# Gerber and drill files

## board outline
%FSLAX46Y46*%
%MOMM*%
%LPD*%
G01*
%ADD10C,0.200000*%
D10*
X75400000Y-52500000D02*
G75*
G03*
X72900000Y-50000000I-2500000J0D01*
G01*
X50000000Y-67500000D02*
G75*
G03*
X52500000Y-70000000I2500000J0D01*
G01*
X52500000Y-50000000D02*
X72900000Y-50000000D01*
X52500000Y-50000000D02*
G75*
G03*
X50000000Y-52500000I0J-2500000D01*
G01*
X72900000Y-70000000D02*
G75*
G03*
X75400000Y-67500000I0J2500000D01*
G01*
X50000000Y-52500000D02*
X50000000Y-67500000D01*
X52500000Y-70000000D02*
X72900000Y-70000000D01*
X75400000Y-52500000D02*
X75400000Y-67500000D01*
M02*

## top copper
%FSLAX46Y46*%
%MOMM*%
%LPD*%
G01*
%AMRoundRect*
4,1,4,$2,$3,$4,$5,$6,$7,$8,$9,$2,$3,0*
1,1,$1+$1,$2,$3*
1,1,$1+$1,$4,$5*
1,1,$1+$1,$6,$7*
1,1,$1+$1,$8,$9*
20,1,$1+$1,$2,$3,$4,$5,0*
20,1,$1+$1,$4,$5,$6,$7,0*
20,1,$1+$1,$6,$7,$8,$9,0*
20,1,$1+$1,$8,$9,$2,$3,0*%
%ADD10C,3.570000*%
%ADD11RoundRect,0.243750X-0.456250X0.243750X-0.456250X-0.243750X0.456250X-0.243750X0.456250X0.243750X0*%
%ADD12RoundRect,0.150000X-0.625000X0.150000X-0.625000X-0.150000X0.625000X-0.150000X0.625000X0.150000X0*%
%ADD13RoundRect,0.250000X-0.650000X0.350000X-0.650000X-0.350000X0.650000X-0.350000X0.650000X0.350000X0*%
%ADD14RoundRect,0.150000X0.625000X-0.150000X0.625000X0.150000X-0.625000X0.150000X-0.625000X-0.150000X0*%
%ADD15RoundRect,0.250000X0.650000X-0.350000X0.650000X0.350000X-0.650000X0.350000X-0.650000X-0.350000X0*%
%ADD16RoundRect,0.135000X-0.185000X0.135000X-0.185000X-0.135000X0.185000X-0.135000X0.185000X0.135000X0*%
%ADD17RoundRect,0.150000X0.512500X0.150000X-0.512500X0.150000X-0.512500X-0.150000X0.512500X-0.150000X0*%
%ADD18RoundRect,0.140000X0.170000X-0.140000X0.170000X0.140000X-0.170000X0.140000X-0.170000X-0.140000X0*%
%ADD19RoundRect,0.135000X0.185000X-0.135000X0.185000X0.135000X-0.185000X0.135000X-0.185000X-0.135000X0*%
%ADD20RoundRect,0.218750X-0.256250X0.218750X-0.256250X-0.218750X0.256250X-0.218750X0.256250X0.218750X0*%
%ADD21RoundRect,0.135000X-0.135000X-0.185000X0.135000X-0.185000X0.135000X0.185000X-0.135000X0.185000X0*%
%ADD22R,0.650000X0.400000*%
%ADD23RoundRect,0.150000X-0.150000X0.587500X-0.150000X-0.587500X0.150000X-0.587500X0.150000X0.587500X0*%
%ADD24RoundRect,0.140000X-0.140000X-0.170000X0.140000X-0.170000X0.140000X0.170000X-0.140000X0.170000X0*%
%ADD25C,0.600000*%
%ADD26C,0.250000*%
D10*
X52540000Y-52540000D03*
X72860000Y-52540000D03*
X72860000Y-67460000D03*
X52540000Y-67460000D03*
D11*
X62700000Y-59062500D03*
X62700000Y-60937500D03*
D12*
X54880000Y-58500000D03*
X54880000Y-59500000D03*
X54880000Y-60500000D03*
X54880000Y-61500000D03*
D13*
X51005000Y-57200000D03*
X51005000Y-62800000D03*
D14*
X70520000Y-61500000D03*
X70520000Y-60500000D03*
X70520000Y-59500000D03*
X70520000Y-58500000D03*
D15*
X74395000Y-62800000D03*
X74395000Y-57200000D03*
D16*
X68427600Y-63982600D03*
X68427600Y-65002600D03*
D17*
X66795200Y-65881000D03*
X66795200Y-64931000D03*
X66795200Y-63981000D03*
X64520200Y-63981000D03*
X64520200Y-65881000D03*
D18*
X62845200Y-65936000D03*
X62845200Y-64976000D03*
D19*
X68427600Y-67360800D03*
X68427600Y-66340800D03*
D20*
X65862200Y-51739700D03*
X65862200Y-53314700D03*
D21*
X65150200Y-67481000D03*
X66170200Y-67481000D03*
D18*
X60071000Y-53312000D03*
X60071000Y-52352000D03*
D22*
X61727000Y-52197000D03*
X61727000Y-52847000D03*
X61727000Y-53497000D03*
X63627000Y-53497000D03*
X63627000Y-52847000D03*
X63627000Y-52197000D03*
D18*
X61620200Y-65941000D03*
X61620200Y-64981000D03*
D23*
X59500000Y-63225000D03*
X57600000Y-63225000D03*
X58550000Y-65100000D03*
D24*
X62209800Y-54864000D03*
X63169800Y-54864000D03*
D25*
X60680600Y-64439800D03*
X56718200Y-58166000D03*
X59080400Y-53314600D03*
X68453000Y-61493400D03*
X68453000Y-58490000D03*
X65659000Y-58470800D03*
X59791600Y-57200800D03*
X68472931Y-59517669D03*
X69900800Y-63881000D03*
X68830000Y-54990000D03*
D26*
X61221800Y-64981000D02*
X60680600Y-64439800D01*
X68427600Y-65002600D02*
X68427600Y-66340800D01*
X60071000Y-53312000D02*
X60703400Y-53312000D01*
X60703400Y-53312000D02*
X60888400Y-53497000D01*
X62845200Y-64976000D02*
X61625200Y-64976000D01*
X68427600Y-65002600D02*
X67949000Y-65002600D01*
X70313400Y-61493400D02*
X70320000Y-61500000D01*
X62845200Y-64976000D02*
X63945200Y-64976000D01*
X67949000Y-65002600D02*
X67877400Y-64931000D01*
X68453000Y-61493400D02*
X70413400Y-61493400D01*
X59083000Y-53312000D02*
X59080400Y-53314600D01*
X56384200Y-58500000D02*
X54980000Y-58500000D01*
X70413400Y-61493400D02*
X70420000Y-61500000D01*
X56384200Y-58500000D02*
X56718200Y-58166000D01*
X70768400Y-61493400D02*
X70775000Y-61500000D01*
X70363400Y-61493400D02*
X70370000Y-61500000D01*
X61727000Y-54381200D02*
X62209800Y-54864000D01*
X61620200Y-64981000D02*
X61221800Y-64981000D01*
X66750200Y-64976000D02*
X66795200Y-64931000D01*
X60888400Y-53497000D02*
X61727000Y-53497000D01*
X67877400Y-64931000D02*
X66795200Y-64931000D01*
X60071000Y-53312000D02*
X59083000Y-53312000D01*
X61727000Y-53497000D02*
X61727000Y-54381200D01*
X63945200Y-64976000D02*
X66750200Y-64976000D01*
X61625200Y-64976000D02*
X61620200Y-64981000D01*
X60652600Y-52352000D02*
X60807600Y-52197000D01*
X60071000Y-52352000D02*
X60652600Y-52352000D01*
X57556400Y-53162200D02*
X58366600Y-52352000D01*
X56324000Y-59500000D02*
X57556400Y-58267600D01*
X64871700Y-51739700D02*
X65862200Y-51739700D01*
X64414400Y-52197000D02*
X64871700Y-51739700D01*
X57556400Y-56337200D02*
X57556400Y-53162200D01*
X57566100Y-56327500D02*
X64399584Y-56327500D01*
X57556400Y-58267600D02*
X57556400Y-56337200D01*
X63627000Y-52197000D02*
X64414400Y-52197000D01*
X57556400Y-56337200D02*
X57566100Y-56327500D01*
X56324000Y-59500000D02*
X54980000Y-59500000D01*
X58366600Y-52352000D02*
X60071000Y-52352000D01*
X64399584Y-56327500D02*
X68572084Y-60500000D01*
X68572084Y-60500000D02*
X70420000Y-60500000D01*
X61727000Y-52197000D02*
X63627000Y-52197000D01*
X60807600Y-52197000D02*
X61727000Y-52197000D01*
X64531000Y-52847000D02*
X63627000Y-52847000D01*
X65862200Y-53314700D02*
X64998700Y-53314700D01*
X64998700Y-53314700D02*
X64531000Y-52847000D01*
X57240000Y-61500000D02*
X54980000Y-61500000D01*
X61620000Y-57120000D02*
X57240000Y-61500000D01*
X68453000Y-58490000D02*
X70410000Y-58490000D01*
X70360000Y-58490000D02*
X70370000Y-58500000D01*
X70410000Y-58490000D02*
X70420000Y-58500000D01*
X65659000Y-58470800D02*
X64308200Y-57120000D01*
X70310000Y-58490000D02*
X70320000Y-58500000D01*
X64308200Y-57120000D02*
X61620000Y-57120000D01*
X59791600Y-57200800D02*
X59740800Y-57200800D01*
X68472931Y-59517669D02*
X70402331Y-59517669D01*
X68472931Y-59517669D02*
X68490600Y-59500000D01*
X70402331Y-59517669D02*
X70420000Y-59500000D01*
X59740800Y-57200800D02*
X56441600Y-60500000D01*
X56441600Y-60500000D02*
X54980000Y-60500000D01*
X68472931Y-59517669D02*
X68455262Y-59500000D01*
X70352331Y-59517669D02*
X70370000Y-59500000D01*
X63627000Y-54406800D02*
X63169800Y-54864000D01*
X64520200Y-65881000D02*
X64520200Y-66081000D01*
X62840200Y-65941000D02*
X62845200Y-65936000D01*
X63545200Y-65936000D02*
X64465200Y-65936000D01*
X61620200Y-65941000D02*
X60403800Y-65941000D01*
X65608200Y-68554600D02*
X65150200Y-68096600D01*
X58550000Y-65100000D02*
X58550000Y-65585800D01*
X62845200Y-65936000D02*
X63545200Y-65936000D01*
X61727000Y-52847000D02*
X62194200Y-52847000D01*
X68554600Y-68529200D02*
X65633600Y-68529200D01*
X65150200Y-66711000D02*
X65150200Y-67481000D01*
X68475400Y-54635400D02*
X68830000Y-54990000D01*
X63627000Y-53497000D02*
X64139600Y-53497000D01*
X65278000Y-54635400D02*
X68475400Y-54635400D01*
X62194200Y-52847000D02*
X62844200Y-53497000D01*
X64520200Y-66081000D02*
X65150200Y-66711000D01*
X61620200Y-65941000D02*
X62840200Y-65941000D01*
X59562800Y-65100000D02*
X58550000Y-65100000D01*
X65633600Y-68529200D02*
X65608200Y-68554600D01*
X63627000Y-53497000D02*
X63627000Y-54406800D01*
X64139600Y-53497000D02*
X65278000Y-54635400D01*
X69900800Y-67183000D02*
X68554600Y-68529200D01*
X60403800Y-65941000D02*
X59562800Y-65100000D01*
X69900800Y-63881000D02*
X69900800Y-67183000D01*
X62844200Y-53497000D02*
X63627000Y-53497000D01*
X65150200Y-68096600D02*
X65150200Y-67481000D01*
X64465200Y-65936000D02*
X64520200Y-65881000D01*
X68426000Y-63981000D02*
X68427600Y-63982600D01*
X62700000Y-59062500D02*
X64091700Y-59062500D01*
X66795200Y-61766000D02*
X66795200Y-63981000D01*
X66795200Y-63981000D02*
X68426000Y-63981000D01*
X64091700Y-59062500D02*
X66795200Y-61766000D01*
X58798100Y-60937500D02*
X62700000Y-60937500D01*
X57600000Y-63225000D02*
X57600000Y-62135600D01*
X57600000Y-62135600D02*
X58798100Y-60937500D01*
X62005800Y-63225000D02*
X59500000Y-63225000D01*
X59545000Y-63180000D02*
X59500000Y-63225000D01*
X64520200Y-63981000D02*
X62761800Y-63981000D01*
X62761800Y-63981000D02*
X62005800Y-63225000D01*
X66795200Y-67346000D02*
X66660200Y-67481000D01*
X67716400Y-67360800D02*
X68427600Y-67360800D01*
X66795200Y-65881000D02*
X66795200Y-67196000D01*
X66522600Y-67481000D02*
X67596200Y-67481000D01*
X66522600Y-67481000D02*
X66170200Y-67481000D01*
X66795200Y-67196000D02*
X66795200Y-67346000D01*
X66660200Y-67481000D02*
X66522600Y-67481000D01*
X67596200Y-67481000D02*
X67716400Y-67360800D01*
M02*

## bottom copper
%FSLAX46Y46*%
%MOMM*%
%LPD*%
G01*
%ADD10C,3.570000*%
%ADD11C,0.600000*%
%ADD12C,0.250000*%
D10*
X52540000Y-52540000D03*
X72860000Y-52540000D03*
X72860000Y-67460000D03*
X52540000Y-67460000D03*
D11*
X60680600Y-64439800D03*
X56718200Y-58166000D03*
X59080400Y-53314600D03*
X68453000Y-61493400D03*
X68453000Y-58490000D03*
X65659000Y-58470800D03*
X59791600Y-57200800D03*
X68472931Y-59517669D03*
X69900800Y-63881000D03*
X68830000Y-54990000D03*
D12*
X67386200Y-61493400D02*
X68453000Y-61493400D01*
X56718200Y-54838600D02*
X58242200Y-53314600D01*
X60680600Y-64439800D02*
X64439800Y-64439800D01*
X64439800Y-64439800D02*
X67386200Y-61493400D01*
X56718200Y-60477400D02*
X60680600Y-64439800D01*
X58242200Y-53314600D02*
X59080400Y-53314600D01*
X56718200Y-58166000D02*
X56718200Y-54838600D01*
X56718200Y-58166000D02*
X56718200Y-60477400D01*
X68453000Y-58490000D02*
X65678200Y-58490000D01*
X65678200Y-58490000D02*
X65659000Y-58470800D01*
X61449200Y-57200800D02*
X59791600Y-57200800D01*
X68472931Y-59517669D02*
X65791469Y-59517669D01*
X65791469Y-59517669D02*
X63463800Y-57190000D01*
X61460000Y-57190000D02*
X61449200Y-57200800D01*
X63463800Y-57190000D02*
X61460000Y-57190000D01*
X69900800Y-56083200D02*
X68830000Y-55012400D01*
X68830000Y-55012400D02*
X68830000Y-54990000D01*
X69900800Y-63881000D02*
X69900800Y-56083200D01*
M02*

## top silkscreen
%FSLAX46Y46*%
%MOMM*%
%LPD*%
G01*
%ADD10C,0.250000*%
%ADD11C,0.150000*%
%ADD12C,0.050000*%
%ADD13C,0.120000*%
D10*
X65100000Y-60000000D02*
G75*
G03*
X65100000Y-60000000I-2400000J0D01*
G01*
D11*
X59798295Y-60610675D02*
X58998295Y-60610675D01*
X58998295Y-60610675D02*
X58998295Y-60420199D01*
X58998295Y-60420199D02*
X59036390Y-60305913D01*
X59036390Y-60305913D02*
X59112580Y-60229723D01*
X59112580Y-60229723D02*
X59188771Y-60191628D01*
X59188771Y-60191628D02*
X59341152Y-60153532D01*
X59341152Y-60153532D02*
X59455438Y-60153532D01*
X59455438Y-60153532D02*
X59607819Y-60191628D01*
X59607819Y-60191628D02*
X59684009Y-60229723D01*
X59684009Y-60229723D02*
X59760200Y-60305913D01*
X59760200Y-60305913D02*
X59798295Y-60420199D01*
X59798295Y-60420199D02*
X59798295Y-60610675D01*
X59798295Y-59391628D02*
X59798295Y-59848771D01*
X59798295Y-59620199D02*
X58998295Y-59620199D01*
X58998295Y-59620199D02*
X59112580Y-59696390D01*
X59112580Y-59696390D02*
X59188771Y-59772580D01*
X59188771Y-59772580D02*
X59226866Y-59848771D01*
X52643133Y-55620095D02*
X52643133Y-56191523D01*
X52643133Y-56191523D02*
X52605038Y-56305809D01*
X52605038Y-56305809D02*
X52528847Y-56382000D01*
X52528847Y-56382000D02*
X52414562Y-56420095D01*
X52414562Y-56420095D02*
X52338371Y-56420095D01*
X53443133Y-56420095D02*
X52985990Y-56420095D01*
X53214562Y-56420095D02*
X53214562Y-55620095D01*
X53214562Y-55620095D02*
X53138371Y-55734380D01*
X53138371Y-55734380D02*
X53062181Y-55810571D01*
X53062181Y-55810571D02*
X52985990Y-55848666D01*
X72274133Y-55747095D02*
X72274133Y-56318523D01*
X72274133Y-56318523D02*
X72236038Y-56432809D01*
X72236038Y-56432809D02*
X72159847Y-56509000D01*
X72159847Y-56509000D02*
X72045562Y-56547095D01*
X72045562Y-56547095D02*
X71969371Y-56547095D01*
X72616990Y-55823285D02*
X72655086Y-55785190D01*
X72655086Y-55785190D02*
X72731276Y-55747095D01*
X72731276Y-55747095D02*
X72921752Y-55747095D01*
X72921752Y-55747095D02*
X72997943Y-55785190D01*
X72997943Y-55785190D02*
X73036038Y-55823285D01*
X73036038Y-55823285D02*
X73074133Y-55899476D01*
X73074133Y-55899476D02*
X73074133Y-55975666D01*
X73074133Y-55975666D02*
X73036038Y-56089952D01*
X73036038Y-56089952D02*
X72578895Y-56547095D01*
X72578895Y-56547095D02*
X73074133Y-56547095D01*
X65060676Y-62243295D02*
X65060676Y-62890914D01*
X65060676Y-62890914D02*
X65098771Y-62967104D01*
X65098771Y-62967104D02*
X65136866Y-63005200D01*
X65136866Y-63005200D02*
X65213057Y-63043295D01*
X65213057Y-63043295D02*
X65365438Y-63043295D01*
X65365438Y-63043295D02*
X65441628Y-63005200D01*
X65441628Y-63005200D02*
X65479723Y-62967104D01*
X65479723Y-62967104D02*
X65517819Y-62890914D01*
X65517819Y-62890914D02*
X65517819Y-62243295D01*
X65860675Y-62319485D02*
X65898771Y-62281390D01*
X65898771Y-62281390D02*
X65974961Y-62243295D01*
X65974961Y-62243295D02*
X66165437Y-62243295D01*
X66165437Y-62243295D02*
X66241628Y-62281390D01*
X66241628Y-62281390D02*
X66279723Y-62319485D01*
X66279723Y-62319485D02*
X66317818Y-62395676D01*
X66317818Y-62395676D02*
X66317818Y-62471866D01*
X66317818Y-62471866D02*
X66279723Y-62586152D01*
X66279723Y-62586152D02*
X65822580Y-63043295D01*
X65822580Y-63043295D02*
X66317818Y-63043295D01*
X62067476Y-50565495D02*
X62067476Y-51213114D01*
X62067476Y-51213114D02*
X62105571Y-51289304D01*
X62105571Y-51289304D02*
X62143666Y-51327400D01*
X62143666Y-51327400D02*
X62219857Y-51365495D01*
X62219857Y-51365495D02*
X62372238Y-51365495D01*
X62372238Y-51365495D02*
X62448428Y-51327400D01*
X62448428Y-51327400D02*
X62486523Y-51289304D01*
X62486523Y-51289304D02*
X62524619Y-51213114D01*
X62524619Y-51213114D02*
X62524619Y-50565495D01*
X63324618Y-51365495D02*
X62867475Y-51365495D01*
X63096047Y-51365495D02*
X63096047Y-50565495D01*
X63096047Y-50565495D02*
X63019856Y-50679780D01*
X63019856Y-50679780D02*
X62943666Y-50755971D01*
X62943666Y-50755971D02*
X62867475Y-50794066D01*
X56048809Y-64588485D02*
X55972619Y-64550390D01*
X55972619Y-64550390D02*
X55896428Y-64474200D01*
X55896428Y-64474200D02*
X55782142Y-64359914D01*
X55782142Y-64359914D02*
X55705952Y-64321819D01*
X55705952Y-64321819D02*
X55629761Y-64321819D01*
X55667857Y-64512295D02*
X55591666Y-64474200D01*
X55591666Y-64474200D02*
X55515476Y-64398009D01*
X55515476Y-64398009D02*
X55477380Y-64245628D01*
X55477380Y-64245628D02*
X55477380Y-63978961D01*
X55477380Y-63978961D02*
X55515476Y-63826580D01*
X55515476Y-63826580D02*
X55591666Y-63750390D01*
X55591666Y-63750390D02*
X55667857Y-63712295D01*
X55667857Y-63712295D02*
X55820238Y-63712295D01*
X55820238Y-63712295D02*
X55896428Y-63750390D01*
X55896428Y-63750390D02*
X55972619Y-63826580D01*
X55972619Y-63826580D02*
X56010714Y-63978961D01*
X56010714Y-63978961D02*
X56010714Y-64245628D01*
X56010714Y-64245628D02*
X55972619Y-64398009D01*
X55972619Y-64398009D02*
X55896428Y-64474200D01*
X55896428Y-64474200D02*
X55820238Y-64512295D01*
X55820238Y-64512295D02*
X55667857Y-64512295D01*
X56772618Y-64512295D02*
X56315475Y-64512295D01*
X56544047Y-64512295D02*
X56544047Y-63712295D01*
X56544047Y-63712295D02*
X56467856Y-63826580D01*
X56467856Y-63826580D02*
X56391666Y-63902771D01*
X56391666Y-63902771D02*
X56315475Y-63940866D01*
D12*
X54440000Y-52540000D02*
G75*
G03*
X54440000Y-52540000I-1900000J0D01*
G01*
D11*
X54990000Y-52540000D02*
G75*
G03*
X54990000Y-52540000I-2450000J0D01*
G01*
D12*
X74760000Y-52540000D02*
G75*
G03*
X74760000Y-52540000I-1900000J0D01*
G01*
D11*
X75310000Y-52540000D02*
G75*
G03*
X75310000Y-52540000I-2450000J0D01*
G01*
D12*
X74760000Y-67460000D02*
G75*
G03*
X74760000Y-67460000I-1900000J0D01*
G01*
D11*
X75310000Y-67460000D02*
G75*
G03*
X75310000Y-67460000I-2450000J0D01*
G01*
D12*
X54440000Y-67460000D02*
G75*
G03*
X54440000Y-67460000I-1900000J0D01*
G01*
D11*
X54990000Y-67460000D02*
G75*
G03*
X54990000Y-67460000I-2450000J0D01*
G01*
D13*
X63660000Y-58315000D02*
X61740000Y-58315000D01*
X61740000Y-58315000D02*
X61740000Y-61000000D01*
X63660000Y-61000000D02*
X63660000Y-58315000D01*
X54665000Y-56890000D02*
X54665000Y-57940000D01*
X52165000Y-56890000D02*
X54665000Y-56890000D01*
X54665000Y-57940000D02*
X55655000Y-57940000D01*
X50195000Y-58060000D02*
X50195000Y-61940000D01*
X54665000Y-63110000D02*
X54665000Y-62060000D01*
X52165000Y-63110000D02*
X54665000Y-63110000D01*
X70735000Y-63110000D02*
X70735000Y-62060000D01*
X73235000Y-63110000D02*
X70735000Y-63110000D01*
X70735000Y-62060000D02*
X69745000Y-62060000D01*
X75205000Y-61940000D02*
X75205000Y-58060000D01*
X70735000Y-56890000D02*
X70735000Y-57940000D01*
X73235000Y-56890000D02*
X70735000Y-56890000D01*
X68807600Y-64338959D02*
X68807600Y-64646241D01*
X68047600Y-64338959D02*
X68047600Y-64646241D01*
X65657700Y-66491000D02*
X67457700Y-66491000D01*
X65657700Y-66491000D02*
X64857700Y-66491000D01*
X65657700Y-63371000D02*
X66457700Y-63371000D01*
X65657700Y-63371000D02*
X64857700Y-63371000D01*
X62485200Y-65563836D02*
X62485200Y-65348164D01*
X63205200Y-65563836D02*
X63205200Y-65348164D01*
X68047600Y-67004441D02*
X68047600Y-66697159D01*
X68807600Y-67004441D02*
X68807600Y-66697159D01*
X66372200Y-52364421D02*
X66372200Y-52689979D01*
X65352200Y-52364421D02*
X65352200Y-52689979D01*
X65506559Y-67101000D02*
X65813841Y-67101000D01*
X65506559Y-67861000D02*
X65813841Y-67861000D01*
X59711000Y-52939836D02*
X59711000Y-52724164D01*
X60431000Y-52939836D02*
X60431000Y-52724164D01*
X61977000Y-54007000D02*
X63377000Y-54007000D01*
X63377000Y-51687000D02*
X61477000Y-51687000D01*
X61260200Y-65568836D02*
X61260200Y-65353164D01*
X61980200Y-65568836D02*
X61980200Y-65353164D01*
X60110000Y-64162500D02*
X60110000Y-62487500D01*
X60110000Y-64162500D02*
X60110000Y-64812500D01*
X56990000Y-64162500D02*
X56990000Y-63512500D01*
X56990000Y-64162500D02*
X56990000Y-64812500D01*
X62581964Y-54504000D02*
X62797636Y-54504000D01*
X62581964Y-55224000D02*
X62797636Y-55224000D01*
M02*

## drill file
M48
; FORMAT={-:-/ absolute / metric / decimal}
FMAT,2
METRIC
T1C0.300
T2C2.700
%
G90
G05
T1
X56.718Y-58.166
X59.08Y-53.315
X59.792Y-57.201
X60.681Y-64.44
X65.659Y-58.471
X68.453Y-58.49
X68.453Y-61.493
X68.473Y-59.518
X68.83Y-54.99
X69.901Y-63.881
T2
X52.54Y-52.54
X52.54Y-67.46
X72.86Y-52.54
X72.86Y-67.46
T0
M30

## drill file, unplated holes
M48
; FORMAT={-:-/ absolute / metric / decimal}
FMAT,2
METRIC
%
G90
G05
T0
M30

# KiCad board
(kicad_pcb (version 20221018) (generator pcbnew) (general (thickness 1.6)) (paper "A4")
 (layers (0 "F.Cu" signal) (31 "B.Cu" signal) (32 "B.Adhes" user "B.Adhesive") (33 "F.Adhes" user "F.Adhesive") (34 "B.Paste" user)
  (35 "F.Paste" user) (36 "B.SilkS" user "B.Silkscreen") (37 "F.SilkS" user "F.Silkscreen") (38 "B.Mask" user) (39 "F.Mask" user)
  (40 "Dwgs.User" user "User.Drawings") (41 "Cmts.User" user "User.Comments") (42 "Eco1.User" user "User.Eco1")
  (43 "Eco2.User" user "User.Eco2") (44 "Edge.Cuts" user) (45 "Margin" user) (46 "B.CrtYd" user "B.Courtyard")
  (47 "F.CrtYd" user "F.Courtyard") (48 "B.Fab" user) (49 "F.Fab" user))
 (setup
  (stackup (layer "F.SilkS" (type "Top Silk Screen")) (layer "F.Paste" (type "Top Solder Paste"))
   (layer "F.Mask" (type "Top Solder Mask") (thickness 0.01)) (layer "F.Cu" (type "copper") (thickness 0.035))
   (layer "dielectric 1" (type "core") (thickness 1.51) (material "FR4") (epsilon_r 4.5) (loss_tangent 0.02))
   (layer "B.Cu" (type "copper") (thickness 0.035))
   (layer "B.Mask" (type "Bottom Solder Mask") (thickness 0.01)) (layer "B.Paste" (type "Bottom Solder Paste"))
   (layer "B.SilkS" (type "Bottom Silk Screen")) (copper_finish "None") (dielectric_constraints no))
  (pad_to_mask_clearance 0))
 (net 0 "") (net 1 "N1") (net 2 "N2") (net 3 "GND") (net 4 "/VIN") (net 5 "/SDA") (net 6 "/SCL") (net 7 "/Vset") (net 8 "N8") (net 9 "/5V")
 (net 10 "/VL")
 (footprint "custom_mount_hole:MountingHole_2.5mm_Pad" (layer "F.Cu") (at 52.54 52.54)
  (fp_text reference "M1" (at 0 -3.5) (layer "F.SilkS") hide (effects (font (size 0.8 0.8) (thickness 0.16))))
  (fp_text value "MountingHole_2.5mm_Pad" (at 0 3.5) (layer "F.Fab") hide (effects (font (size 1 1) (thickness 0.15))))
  (fp_circle (center 0 0) (end 1.9 0) (stroke (width 0.05) (type solid)) (fill none) (layer "F.SilkS"))
  (fp_circle (center 0 0) (end 2.45 0) (stroke (width 0.15) (type solid)) (fill none) (layer "F.SilkS"))
  (pad "~" thru_hole circle (at 0 0) (size 3.57 3.57) (drill 2.7) (layers "*.Cu" "*.Mask")))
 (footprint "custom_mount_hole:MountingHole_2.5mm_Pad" (layer "F.Cu") (at 72.86 52.54)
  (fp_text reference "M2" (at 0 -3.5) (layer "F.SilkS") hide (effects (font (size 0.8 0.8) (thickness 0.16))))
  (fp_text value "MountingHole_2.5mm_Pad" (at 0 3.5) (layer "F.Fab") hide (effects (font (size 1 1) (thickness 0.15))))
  (fp_circle (center 0 0) (end 1.9 0) (stroke (width 0.05) (type solid)) (fill none) (layer "F.SilkS"))
  (fp_circle (center 0 0) (end 2.45 0) (stroke (width 0.15) (type solid)) (fill none) (layer "F.SilkS"))
  (pad "~" thru_hole circle (at 0 0) (size 3.57 3.57) (drill 2.7) (layers "*.Cu" "*.Mask")))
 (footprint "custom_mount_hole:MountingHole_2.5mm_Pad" (layer "F.Cu") (at 72.86 67.46)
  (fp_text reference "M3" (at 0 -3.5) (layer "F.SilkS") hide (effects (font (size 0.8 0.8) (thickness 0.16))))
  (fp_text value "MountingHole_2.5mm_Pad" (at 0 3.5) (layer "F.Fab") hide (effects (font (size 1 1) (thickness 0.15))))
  (fp_circle (center 0 0) (end 1.9 0) (stroke (width 0.05) (type solid)) (fill none) (layer "F.SilkS"))
  (fp_circle (center 0 0) (end 2.45 0) (stroke (width 0.15) (type solid)) (fill none) (layer "F.SilkS"))
  (pad "~" thru_hole circle (at 0 0) (size 3.57 3.57) (drill 2.7) (layers "*.Cu" "*.Mask")))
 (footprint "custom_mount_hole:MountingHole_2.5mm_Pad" (layer "F.Cu") (at 52.54 67.46)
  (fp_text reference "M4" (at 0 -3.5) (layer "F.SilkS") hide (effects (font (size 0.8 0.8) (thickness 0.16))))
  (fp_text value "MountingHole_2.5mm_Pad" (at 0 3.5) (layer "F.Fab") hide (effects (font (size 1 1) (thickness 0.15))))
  (fp_circle (center 0 0) (end 1.9 0) (stroke (width 0.05) (type solid)) (fill none) (layer "F.SilkS"))
  (fp_circle (center 0 0) (end 2.45 0) (stroke (width 0.15) (type solid)) (fill none) (layer "F.SilkS"))
  (pad "~" thru_hole circle (at 0 0) (size 3.57 3.57) (drill 2.7) (layers "*.Cu" "*.Mask")))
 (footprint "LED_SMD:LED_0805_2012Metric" (layer "F.Cu") (at 62.7 60 -90)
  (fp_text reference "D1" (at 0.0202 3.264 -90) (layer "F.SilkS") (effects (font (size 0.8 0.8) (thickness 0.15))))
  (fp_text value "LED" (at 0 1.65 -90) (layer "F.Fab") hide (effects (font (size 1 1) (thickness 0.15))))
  (fp_line (start -1.685 -0.96) (end -1.685 0.96) (stroke (width 0.12) (type solid)) (layer "F.SilkS"))
  (fp_line (start -1.685 0.96) (end 1 0.96) (stroke (width 0.12) (type solid)) (layer "F.SilkS"))
  (fp_line (start 1 -0.96) (end -1.685 -0.96) (stroke (width 0.12) (type solid)) (layer "F.SilkS"))
  (pad "1" smd roundrect (at -0.9375 0 270) (size 0.975 1.4) (layers "F.Cu" "F.Paste" "F.Mask") (roundrect_rratio 0.25) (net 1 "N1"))
  (pad "2" smd roundrect (at 0.9375 0 270) (size 0.975 1.4) (layers "F.Cu" "F.Paste" "F.Mask") (roundrect_rratio 0.25) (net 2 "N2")))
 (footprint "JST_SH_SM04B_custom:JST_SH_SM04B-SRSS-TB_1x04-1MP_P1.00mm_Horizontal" (layer "F.Cu") (at 52.88 60 -90)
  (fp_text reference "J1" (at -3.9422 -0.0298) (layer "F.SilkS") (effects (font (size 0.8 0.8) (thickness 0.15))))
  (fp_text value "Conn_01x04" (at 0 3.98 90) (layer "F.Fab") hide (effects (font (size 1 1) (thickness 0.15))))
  (fp_line (start -3.11 -1.785) (end -2.06 -1.785) (stroke (width 0.12) (type solid)) (layer "F.SilkS"))
  (fp_line (start -3.11 0.715) (end -3.11 -1.785) (stroke (width 0.12) (type solid)) (layer "F.SilkS"))
  (fp_line (start -2.06 -1.785) (end -2.06 -2.775) (stroke (width 0.12) (type solid)) (layer "F.SilkS"))
  (fp_line (start -1.94 2.685) (end 1.94 2.685) (stroke (width 0.12) (type solid)) (layer "F.SilkS"))
  (fp_line (start 3.11 -1.785) (end 2.06 -1.785) (stroke (width 0.12) (type solid)) (layer "F.SilkS"))
  (fp_line (start 3.11 0.715) (end 3.11 -1.785) (stroke (width 0.12) (type solid)) (layer "F.SilkS"))
  (pad "1" smd roundrect (at -1.5 -2 270) (size 0.6 1.55) (layers "F.Cu" "F.Paste" "F.Mask") (roundrect_rratio 0.25) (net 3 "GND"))
  (pad "2" smd roundrect (at -0.5 -2 270) (size 0.6 1.55) (layers "F.Cu" "F.Paste" "F.Mask") (roundrect_rratio 0.25) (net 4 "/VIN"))
  (pad "3" smd roundrect (at 0.5 -2 270) (size 0.6 1.55) (layers "F.Cu" "F.Paste" "F.Mask") (roundrect_rratio 0.25) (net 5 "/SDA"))
  (pad "4" smd roundrect (at 1.5 -2 270) (size 0.6 1.55) (layers "F.Cu" "F.Paste" "F.Mask") (roundrect_rratio 0.25) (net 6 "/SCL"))
  (pad "MP" smd roundrect (at -2.8 1.875 270) (size 1.2 1.8) (layers "F.Cu" "F.Paste" "F.Mask") (roundrect_rratio 0.2083333333))
  (pad "MP" smd roundrect (at 2.8 1.875 270) (size 1.2 1.8) (layers "F.Cu" "F.Paste" "F.Mask") (roundrect_rratio 0.2083333333)))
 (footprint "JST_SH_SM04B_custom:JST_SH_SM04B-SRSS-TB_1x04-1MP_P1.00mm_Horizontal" (layer "F.Cu") (at 72.52 60 90)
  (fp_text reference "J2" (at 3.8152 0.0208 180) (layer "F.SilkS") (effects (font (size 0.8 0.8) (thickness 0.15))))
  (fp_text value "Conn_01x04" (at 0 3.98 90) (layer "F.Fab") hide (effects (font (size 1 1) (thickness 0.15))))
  (fp_line (start -3.11 -1.785) (end -2.06 -1.785) (stroke (width 0.12) (type solid)) (layer "F.SilkS"))
  (fp_line (start -3.11 0.715) (end -3.11 -1.785) (stroke (width 0.12) (type solid)) (layer "F.SilkS"))
  (fp_line (start -2.06 -1.785) (end -2.06 -2.775) (stroke (width 0.12) (type solid)) (layer "F.SilkS"))
  (fp_line (start -1.94 2.685) (end 1.94 2.685) (stroke (width 0.12) (type solid)) (layer "F.SilkS"))
  (fp_line (start 3.11 -1.785) (end 2.06 -1.785) (stroke (width 0.12) (type solid)) (layer "F.SilkS"))
  (fp_line (start 3.11 0.715) (end 3.11 -1.785) (stroke (width 0.12) (type solid)) (layer "F.SilkS"))
  (pad "1" smd roundrect (at -1.5 -2 90) (size 0.6 1.55) (layers "F.Cu" "F.Paste" "F.Mask") (roundrect_rratio 0.25) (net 3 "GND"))
  (pad "2" smd roundrect (at -0.5 -2 90) (size 0.6 1.55) (layers "F.Cu" "F.Paste" "F.Mask") (roundrect_rratio 0.25) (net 4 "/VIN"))
  (pad "3" smd roundrect (at 0.5 -2 90) (size 0.6 1.55) (layers "F.Cu" "F.Paste" "F.Mask") (roundrect_rratio 0.25) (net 5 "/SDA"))
  (pad "4" smd roundrect (at 1.5 -2 90) (size 0.6 1.55) (layers "F.Cu" "F.Paste" "F.Mask") (roundrect_rratio 0.25) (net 6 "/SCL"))
  (pad "MP" smd roundrect (at -2.8 1.875 90) (size 1.2 1.8) (layers "F.Cu" "F.Paste" "F.Mask") (roundrect_rratio 0.2083333333))
  (pad "MP" smd roundrect (at 2.8 1.875 90) (size 1.2 1.8) (layers "F.Cu" "F.Paste" "F.Mask") (roundrect_rratio 0.2083333333)))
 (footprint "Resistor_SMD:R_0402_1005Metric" (layer "F.Cu") (at 68.4276 64.4926 -90)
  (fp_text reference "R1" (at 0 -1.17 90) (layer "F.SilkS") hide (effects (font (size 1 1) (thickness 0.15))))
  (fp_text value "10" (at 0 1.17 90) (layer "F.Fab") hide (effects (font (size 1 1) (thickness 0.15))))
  (fp_line (start -0.153641 -0.38) (end 0.153641 -0.38) (stroke (width 0.12) (type solid)) (layer "F.SilkS"))
  (fp_line (start -0.153641 0.38) (end 0.153641 0.38) (stroke (width 0.12) (type solid)) (layer "F.SilkS"))
  (pad "1" smd roundrect (at -0.51 0 270) (size 0.54 0.64) (layers "F.Cu" "F.Paste" "F.Mask") (roundrect_rratio 0.25) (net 1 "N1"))
  (pad "2" smd roundrect (at 0.51 0 270) (size 0.54 0.64) (layers "F.Cu" "F.Paste" "F.Mask") (roundrect_rratio 0.25) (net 3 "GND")))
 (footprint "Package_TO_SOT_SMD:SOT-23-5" (layer "F.Cu") (at 65.6577 64.931 180)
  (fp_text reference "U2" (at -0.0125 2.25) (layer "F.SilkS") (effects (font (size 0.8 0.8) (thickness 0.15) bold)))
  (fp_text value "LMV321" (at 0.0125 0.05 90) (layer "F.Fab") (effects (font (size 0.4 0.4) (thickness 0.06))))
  (fp_line (start 0 -1.56) (end -1.8 -1.56) (stroke (width 0.12) (type solid)) (layer "F.SilkS"))
  (fp_line (start 0 -1.56) (end 0.8 -1.56) (stroke (width 0.12) (type solid)) (layer "F.SilkS"))
  (fp_line (start 0 1.56) (end -0.8 1.56) (stroke (width 0.12) (type solid)) (layer "F.SilkS"))
  (fp_line (start 0 1.56) (end 0.8 1.56) (stroke (width 0.12) (type solid)) (layer "F.SilkS"))
  (pad "1" smd roundrect (at -1.1375 -0.95 180) (size 1.325 0.6) (layers "F.Cu" "F.Paste" "F.Mask") (roundrect_rratio 0.25) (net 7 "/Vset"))
  (pad "2" smd roundrect (at -1.1375 0 180) (size 1.325 0.6) (layers "F.Cu" "F.Paste" "F.Mask") (roundrect_rratio 0.25) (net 3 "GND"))
  (pad "3" smd roundrect (at -1.1375 0.95 180) (size 1.325 0.6) (layers "F.Cu" "F.Paste" "F.Mask") (roundrect_rratio 0.25) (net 1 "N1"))
  (pad "4" smd roundrect (at 1.1375 0.95 180) (size 1.325 0.6) (layers "F.Cu" "F.Paste" "F.Mask") (roundrect_rratio 0.25) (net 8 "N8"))
  (pad "5" smd roundrect (at 1.1375 -0.95 180) (size 1.325 0.6) (layers "F.Cu" "F.Paste" "F.Mask") (roundrect_rratio 0.25) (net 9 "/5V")))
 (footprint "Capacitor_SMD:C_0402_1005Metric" (layer "F.Cu") (at 62.8452 65.456 90)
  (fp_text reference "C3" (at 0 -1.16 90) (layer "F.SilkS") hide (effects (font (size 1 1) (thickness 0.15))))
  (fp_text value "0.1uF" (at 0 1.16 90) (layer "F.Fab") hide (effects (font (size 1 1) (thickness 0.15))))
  (fp_line (start -0.107836 -0.36) (end 0.107836 -0.36) (stroke (width 0.12) (type solid)) (layer "F.SilkS"))
  (fp_line (start -0.107836 0.36) (end 0.107836 0.36) (stroke (width 0.12) (type solid)) (layer "F.SilkS"))
  (pad "1" smd roundrect (at -0.48 0 90) (size 0.56 0.62) (layers "F.Cu" "F.Paste" "F.Mask") (roundrect_rratio 0.25) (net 9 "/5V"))
  (pad "2" smd roundrect (at 0.48 0 90) (size 0.56 0.62) (layers "F.Cu" "F.Paste" "F.Mask") (roundrect_rratio 0.25) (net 3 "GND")))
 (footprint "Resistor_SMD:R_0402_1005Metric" (layer "F.Cu") (at 68.4276 66.8508 90)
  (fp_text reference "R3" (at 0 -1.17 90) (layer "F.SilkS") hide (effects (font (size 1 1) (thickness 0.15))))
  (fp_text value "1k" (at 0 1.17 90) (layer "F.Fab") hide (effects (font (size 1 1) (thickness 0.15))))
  (fp_line (start -0.153641 -0.38) (end 0.153641 -0.38) (stroke (width 0.12) (type solid)) (layer "F.SilkS"))
  (fp_line (start -0.153641 0.38) (end 0.153641 0.38) (stroke (width 0.12) (type solid)) (layer "F.SilkS"))
  (pad "1" smd roundrect (at -0.51 0 90) (size 0.54 0.64) (layers "F.Cu" "F.Paste" "F.Mask") (roundrect_rratio 0.25) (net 7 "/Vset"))
  (pad "2" smd roundrect (at 0.51 0 90) (size 0.54 0.64) (layers "F.Cu" "F.Paste" "F.Mask") (roundrect_rratio 0.25) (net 3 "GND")))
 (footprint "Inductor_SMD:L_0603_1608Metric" (layer "F.Cu") (at 65.8622 52.5272 -90)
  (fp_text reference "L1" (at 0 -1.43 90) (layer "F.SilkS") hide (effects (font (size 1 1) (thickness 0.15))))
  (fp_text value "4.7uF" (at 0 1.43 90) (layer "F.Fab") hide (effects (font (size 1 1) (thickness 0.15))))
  (fp_line (start -0.162779 -0.51) (end 0.162779 -0.51) (stroke (width 0.12) (type solid)) (layer "F.SilkS"))
  (fp_line (start -0.162779 0.51) (end 0.162779 0.51) (stroke (width 0.12) (type solid)) (layer "F.SilkS"))
  (pad "1" smd roundrect (at -0.7875 0 270) (size 0.875 0.95) (layers "F.Cu" "F.Paste" "F.Mask") (roundrect_rratio 0.25) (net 4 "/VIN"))
  (pad "2" smd roundrect (at 0.7875 0 270) (size 0.875 0.95) (layers "F.Cu" "F.Paste" "F.Mask") (roundrect_rratio 0.25) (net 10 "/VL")))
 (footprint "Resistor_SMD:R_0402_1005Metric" (layer "F.Cu") (at 65.6602 67.481)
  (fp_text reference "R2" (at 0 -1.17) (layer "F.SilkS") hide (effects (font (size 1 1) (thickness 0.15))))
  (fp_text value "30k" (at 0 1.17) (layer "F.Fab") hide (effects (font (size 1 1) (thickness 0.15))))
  (fp_line (start -0.153641 -0.38) (end 0.153641 -0.38) (stroke (width 0.12) (type solid)) (layer "F.SilkS"))
  (fp_line (start -0.153641 0.38) (end 0.153641 0.38) (stroke (width 0.12) (type solid)) (layer "F.SilkS"))
  (pad "1" smd roundrect (at -0.51 0) (size 0.54 0.64) (layers "F.Cu" "F.Paste" "F.Mask") (roundrect_rratio 0.25) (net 9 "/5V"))
  (pad "2" smd roundrect (at 0.51 0) (size 0.54 0.64) (layers "F.Cu" "F.Paste" "F.Mask") (roundrect_rratio 0.25) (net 7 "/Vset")))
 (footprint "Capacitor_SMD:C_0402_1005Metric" (layer "F.Cu") (at 60.071 52.832 90)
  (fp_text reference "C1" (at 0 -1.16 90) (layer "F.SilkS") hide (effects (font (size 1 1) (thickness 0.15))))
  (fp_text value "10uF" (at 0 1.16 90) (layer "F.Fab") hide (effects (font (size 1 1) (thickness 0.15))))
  (fp_line (start -0.107836 -0.36) (end 0.107836 -0.36) (stroke (width 0.12) (type solid)) (layer "F.SilkS"))
  (fp_line (start -0.107836 0.36) (end 0.107836 0.36) (stroke (width 0.12) (type solid)) (layer "F.SilkS"))
  (pad "1" smd roundrect (at -0.48 0 90) (size 0.56 0.62) (layers "F.Cu" "F.Paste" "F.Mask") (roundrect_rratio 0.25) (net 3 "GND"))
  (pad "2" smd roundrect (at 0.48 0 90) (size 0.56 0.62) (layers "F.Cu" "F.Paste" "F.Mask") (roundrect_rratio 0.25) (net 4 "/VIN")))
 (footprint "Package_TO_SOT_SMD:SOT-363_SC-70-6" (layer "F.Cu") (at 62.677 52.847)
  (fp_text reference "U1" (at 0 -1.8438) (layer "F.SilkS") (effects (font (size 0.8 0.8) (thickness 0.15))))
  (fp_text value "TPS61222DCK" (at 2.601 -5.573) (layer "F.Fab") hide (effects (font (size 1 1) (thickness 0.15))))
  (fp_line (start -0.7 1.16) (end 0.7 1.16) (stroke (width 0.12) (type solid)) (layer "F.SilkS"))
  (fp_line (start 0.7 -1.16) (end -1.2 -1.16) (stroke (width 0.12) (type solid)) (layer "F.SilkS"))
  (pad "1" smd rect (at -0.95 -0.65) (size 0.65 0.4) (layers "F.Cu" "F.Paste" "F.Mask") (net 4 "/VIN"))
  (pad "2" smd rect (at -0.95 0) (size 0.65 0.4) (layers "F.Cu" "F.Paste" "F.Mask") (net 9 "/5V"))
  (pad "3" smd rect (at -0.95 0.65) (size 0.65 0.4) (layers "F.Cu" "F.Paste" "F.Mask") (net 3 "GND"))
  (pad "4" smd rect (at 0.95 0.65) (size 0.65 0.4) (layers "F.Cu" "F.Paste" "F.Mask") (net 9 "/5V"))
  (pad "5" smd rect (at 0.95 0) (size 0.65 0.4) (layers "F.Cu" "F.Paste" "F.Mask") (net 10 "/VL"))
  (pad "6" smd rect (at 0.95 -0.65) (size 0.65 0.4) (layers "F.Cu" "F.Paste" "F.Mask") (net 4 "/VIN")))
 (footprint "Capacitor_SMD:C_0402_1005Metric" (layer "F.Cu") (at 61.6202 65.461 90)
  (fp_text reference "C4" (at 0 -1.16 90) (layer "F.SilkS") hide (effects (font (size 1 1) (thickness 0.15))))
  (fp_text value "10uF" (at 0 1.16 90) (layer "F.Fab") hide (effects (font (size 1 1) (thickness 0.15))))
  (fp_line (start -0.107836 -0.36) (end 0.107836 -0.36) (stroke (width 0.12) (type solid)) (layer "F.SilkS"))
  (fp_line (start -0.107836 0.36) (end 0.107836 0.36) (stroke (width 0.12) (type solid)) (layer "F.SilkS"))
  (pad "1" smd roundrect (at -0.48 0 90) (size 0.56 0.62) (layers "F.Cu" "F.Paste" "F.Mask") (roundrect_rratio 0.25) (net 9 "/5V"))
  (pad "2" smd roundrect (at 0.48 0 90) (size 0.56 0.62) (layers "F.Cu" "F.Paste" "F.Mask") (roundrect_rratio 0.25) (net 3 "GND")))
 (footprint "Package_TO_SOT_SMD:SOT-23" (layer "F.Cu") (at 58.55 64.1625 -90)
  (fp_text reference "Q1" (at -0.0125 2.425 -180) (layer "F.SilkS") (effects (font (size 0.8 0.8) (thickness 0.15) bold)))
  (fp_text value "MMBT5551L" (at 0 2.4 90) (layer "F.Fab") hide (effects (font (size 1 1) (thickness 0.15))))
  (fp_line (start 0 -1.56) (end -1.675 -1.56) (stroke (width 0.12) (type solid)) (layer "F.SilkS"))
  (fp_line (start 0 -1.56) (end 0.65 -1.56) (stroke (width 0.12) (type solid)) (layer "F.SilkS"))
  (fp_line (start 0 1.56) (end -0.65 1.56) (stroke (width 0.12) (type solid)) (layer "F.SilkS"))
  (fp_line (start 0 1.56) (end 0.65 1.56) (stroke (width 0.12) (type solid)) (layer "F.SilkS"))
  (pad "1" smd roundrect (at -0.9375 -0.95 270) (size 1.475 0.6) (layers "F.Cu" "F.Paste" "F.Mask") (roundrect_rratio 0.25) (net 8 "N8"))
  (pad "2" smd roundrect (at -0.9375 0.95 270) (size 1.475 0.6) (layers "F.Cu" "F.Paste" "F.Mask") (roundrect_rratio 0.25) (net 2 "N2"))
  (pad "3" smd roundrect (at 0.9375 0 270) (size 1.475 0.6) (layers "F.Cu" "F.Paste" "F.Mask") (roundrect_rratio 0.25) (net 9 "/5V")))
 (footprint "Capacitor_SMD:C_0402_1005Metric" (layer "F.Cu") (at 62.6898 54.864)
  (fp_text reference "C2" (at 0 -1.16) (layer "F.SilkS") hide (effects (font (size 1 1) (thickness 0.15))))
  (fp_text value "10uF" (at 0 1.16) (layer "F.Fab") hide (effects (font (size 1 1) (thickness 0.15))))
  (fp_line (start -0.107836 -0.36) (end 0.107836 -0.36) (stroke (width 0.12) (type solid)) (layer "F.SilkS"))
  (fp_line (start -0.107836 0.36) (end 0.107836 0.36) (stroke (width 0.12) (type solid)) (layer "F.SilkS"))
  (pad "1" smd roundrect (at -0.48 0) (size 0.56 0.62) (layers "F.Cu" "F.Paste" "F.Mask") (roundrect_rratio 0.25) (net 3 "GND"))
  (pad "2" smd roundrect (at 0.48 0) (size 0.56 0.62) (layers "F.Cu" "F.Paste" "F.Mask") (roundrect_rratio 0.25) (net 9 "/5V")))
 (gr_circle (center 62.7 60) (end 65.1 60) (stroke (width 0.25) (type solid)) (fill none) (layer "F.SilkS"))
 (gr_arc (start 72.9 50) (mid 74.667767 50.732233) (end 75.4 52.5) (stroke (width 0.2) (type solid)) (layer "Edge.Cuts"))
 (gr_arc (start 52.5 70) (mid 50.732233 69.267767) (end 50 67.5) (stroke (width 0.2) (type solid)) (layer "Edge.Cuts"))
 (gr_line (start 52.5 50) (end 72.9 50) (stroke (width 0.2) (type solid)) (layer "Edge.Cuts"))
 (gr_arc (start 50 52.5) (mid 50.732233 50.732233) (end 52.5 50) (stroke (width 0.2) (type solid)) (layer "Edge.Cuts"))
 (gr_arc (start 75.4 67.5) (mid 74.667767 69.267767) (end 72.9 70) (stroke (width 0.2) (type solid)) (layer "Edge.Cuts"))
 (gr_line (start 50 52.5) (end 50 67.5) (stroke (width 0.2) (type solid)) (layer "Edge.Cuts"))
 (gr_line (start 52.5 70) (end 72.9 70) (stroke (width 0.2) (type solid)) (layer "Edge.Cuts"))
 (gr_line (start 75.4 52.5) (end 75.4 67.5) (stroke (width 0.2) (type solid)) (layer "Edge.Cuts"))
 (segment (start 61.2218 64.981) (end 60.6806 64.4398) (width 0.25) (layer "F.Cu") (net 3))
 (segment (start 68.4276 65.0026) (end 68.4276 66.3408) (width 0.25) (layer "F.Cu") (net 3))
 (segment (start 60.071 53.312) (end 60.7034 53.312) (width 0.25) (layer "F.Cu") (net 3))
 (segment (start 60.7034 53.312) (end 60.8884 53.497) (width 0.25) (layer "F.Cu") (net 3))
 (segment (start 62.8452 64.976) (end 61.6252 64.976) (width 0.25) (layer "F.Cu") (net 3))
 (segment (start 68.4276 65.0026) (end 67.949 65.0026) (width 0.25) (layer "F.Cu") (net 3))
 (segment (start 70.3134 61.4934) (end 70.32 61.5) (width 0.25) (layer "F.Cu") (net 3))
 (segment (start 62.8452 64.976) (end 63.9452 64.976) (width 0.25) (layer "F.Cu") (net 3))
 (segment (start 67.949 65.0026) (end 67.8774 64.931) (width 0.25) (layer "F.Cu") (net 3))
 (segment (start 68.453 61.4934) (end 70.4134 61.4934) (width 0.25) (layer "F.Cu") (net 3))
 (segment (start 59.083 53.312) (end 59.0804 53.3146) (width 0.25) (layer "F.Cu") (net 3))
 (segment (start 56.3842 58.5) (end 54.98 58.5) (width 0.25) (layer "F.Cu") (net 3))
 (segment (start 70.4134 61.4934) (end 70.42 61.5) (width 0.25) (layer "F.Cu") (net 3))
 (segment (start 56.3842 58.5) (end 56.7182 58.166) (width 0.25) (layer "F.Cu") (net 3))
 (segment (start 70.7684 61.4934) (end 70.775 61.5) (width 0.25) (layer "F.Cu") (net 3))
 (segment (start 70.3634 61.4934) (end 70.37 61.5) (width 0.25) (layer "F.Cu") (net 3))
 (segment (start 61.727 54.3812) (end 62.2098 54.864) (width 0.25) (layer "F.Cu") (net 3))
 (segment (start 61.6202 64.981) (end 61.2218 64.981) (width 0.25) (layer "F.Cu") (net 3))
 (segment (start 66.7502 64.976) (end 66.7952 64.931) (width 0.25) (layer "F.Cu") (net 3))
 (segment (start 60.8884 53.497) (end 61.727 53.497) (width 0.25) (layer "F.Cu") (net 3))
 (segment (start 67.8774 64.931) (end 66.7952 64.931) (width 0.25) (layer "F.Cu") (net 3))
 (segment (start 60.071 53.312) (end 59.083 53.312) (width 0.25) (layer "F.Cu") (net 3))
 (segment (start 61.727 53.497) (end 61.727 54.3812) (width 0.25) (layer "F.Cu") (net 3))
 (segment (start 63.9452 64.976) (end 66.7502 64.976) (width 0.25) (layer "F.Cu") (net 3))
 (segment (start 61.6252 64.976) (end 61.6202 64.981) (width 0.25) (layer "F.Cu") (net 3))
 (via (at 60.6806 64.4398) (size 0.6) (drill 0.3) (layers "F.Cu" "B.Cu") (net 3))
 (via (at 56.7182 58.166) (size 0.6) (drill 0.3) (layers "F.Cu" "B.Cu") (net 3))
 (via (at 59.0804 53.3146) (size 0.6) (drill 0.3) (layers "F.Cu" "B.Cu") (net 3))
 (via (at 68.453 61.4934) (size 0.6) (drill 0.3) (layers "F.Cu" "B.Cu") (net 3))
 (segment (start 67.3862 61.4934) (end 68.453 61.4934) (width 0.25) (layer "B.Cu") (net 3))
 (segment (start 56.7182 54.8386) (end 58.2422 53.3146) (width 0.25) (layer "B.Cu") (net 3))
 (segment (start 60.6806 64.4398) (end 64.4398 64.4398) (width 0.25) (layer "B.Cu") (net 3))
 (segment (start 64.4398 64.4398) (end 67.3862 61.4934) (width 0.25) (layer "B.Cu") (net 3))
 (segment (start 56.7182 60.4774) (end 60.6806 64.4398) (width 0.25) (layer "B.Cu") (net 3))
 (segment (start 58.2422 53.3146) (end 59.0804 53.3146) (width 0.25) (layer "B.Cu") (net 3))
 (segment (start 56.7182 58.166) (end 56.7182 54.8386) (width 0.25) (layer "B.Cu") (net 3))
 (segment (start 56.7182 58.166) (end 56.7182 60.4774) (width 0.25) (layer "B.Cu") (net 3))
 (segment (start 60.6526 52.352) (end 60.8076 52.197) (width 0.25) (layer "F.Cu") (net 4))
 (segment (start 60.071 52.352) (end 60.6526 52.352) (width 0.25) (layer "F.Cu") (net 4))
 (segment (start 57.5564 53.1622) (end 58.3666 52.352) (width 0.25) (layer "F.Cu") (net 4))
 (segment (start 56.324 59.5) (end 57.5564 58.2676) (width 0.25) (layer "F.Cu") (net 4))
 (segment (start 64.8717 51.7397) (end 65.8622 51.7397) (width 0.25) (layer "F.Cu") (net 4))
 (segment (start 64.4144 52.197) (end 64.8717 51.7397) (width 0.25) (layer "F.Cu") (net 4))
 (segment (start 57.5564 56.3372) (end 57.5564 53.1622) (width 0.25) (layer "F.Cu") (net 4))
 (segment (start 57.5661 56.3275) (end 64.399584 56.3275) (width 0.25) (layer "F.Cu") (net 4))
 (segment (start 57.5564 58.2676) (end 57.5564 56.3372) (width 0.25) (layer "F.Cu") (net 4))
 (segment (start 63.627 52.197) (end 64.4144 52.197) (width 0.25) (layer "F.Cu") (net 4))
 (segment (start 57.5564 56.3372) (end 57.5661 56.3275) (width 0.25) (layer "F.Cu") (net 4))
 (segment (start 56.324 59.5) (end 54.98 59.5) (width 0.25) (layer "F.Cu") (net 4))
 (segment (start 58.3666 52.352) (end 60.071 52.352) (width 0.25) (layer "F.Cu") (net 4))
 (segment (start 64.399584 56.3275) (end 68.572084 60.5) (width 0.25) (layer "F.Cu") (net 4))
 (segment (start 68.572084 60.5) (end 70.42 60.5) (width 0.25) (layer "F.Cu") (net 4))
 (segment (start 61.727 52.197) (end 63.627 52.197) (width 0.25) (layer "F.Cu") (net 4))
 (segment (start 60.8076 52.197) (end 61.727 52.197) (width 0.25) (layer "F.Cu") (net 4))
 (segment (start 64.531 52.847) (end 63.627 52.847) (width 0.25) (layer "F.Cu") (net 10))
 (segment (start 65.8622 53.3147) (end 64.9987 53.3147) (width 0.25) (layer "F.Cu") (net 10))
 (segment (start 64.9987 53.3147) (end 64.531 52.847) (width 0.25) (layer "F.Cu") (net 10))
 (segment (start 57.24 61.5) (end 54.98 61.5) (width 0.25) (layer "F.Cu") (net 6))
 (segment (start 61.62 57.12) (end 57.24 61.5) (width 0.25) (layer "F.Cu") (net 6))
 (segment (start 68.453 58.49) (end 70.41 58.49) (width 0.25) (layer "F.Cu") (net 6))
 (segment (start 70.36 58.49) (end 70.37 58.5) (width 0.25) (layer "F.Cu") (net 6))
 (segment (start 70.41 58.49) (end 70.42 58.5) (width 0.25) (layer "F.Cu") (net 6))
 (segment (start 65.659 58.4708) (end 64.3082 57.12) (width 0.25) (layer "F.Cu") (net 6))
 (segment (start 70.31 58.49) (end 70.32 58.5) (width 0.25) (layer "F.Cu") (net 6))
 (segment (start 64.3082 57.12) (end 61.62 57.12) (width 0.25) (layer "F.Cu") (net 6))
 (via (at 68.453 58.49) (size 0.6) (drill 0.3) (layers "F.Cu" "B.Cu") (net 6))
 (via (at 65.659 58.4708) (size 0.6) (drill 0.3) (layers "F.Cu" "B.Cu") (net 6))
 (segment (start 68.453 58.49) (end 65.6782 58.49) (width 0.25) (layer "B.Cu") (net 6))
 (segment (start 65.6782 58.49) (end 65.659 58.4708) (width 0.25) (layer "B.Cu") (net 6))
 (segment (start 59.7916 57.2008) (end 59.7408 57.2008) (width 0.25) (layer "F.Cu") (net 5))
 (segment (start 68.472931 59.517669) (end 70.402331 59.517669) (width 0.25) (layer "F.Cu") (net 5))
 (segment (start 68.472931 59.517669) (end 68.4906 59.5) (width 0.25) (layer "F.Cu") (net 5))
 (segment (start 70.402331 59.517669) (end 70.42 59.5) (width 0.25) (layer "F.Cu") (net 5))
 (segment (start 59.7408 57.2008) (end 56.4416 60.5) (width 0.25) (layer "F.Cu") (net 5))
 (segment (start 56.4416 60.5) (end 54.98 60.5) (width 0.25) (layer "F.Cu") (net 5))
 (segment (start 68.472931 59.517669) (end 68.455262 59.5) (width 0.25) (layer "F.Cu") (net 5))
 (segment (start 70.352331 59.517669) (end 70.37 59.5) (width 0.25) (layer "F.Cu") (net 5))
 (via (at 59.7916 57.2008) (size 0.6) (drill 0.3) (layers "F.Cu" "B.Cu") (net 5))
 (via (at 68.472931 59.517669) (size 0.6) (drill 0.3) (layers "F.Cu" "B.Cu") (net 5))
 (segment (start 61.4492 57.2008) (end 59.7916 57.2008) (width 0.25) (layer "B.Cu") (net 5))
 (segment (start 68.472931 59.517669) (end 65.791469 59.517669) (width 0.25) (layer "B.Cu") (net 5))
 (segment (start 65.791469 59.517669) (end 63.4638 57.19) (width 0.25) (layer "B.Cu") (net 5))
 (segment (start 61.46 57.19) (end 61.4492 57.2008) (width 0.25) (layer "B.Cu") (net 5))
 (segment (start 63.4638 57.19) (end 61.46 57.19) (width 0.25) (layer "B.Cu") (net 5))
 (segment (start 63.627 54.4068) (end 63.1698 54.864) (width 0.25) (layer "F.Cu") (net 9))
 (segment (start 64.5202 65.881) (end 64.5202 66.081) (width 0.25) (layer "F.Cu") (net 9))
 (segment (start 62.8402 65.941) (end 62.8452 65.936) (width 0.25) (layer "F.Cu") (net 9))
 (segment (start 63.5452 65.936) (end 64.4652 65.936) (width 0.25) (layer "F.Cu") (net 9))
 (segment (start 61.6202 65.941) (end 60.4038 65.941) (width 0.25) (layer "F.Cu") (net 9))
 (segment (start 65.6082 68.5546) (end 65.1502 68.0966) (width 0.25) (layer "F.Cu") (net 9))
 (segment (start 58.55 65.1) (end 58.55 65.5858) (width 0.25) (layer "F.Cu") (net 9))
 (segment (start 62.8452 65.936) (end 63.5452 65.936) (width 0.25) (layer "F.Cu") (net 9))
 (segment (start 61.727 52.847) (end 62.1942 52.847) (width 0.25) (layer "F.Cu") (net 9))
 (segment (start 68.5546 68.5292) (end 65.6336 68.5292) (width 0.25) (layer "F.Cu") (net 9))
 (segment (start 65.1502 66.711) (end 65.1502 67.481) (width 0.25) (layer "F.Cu") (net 9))
 (segment (start 68.4754 54.6354) (end 68.83 54.99) (width 0.25) (layer "F.Cu") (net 9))
 (segment (start 63.627 53.497) (end 64.1396 53.497) (width 0.25) (layer "F.Cu") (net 9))
 (segment (start 65.278 54.6354) (end 68.4754 54.6354) (width 0.25) (layer "F.Cu") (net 9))
 (segment (start 62.1942 52.847) (end 62.8442 53.497) (width 0.25) (layer "F.Cu") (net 9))
 (segment (start 64.5202 66.081) (end 65.1502 66.711) (width 0.25) (layer "F.Cu") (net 9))
 (segment (start 61.6202 65.941) (end 62.8402 65.941) (width 0.25) (layer "F.Cu") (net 9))
 (segment (start 59.5628 65.1) (end 58.55 65.1) (width 0.25) (layer "F.Cu") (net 9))
 (segment (start 65.6336 68.5292) (end 65.6082 68.5546) (width 0.25) (layer "F.Cu") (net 9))
 (segment (start 63.627 53.497) (end 63.627 54.4068) (width 0.25) (layer "F.Cu") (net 9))
 (segment (start 64.1396 53.497) (end 65.278 54.6354) (width 0.25) (layer "F.Cu") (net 9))
 (segment (start 69.9008 67.183) (end 68.5546 68.5292) (width 0.25) (layer "F.Cu") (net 9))
 (segment (start 60.4038 65.941) (end 59.5628 65.1) (width 0.25) (layer "F.Cu") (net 9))
 (segment (start 69.9008 63.881) (end 69.9008 67.183) (width 0.25) (layer "F.Cu") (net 9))
 (segment (start 62.8442 53.497) (end 63.627 53.497) (width 0.25) (layer "F.Cu") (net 9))
 (segment (start 65.1502 68.0966) (end 65.1502 67.481) (width 0.25) (layer "F.Cu") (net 9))
 (segment (start 64.4652 65.936) (end 64.5202 65.881) (width 0.25) (layer "F.Cu") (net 9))
 (via (at 69.9008 63.881) (size 0.6) (drill 0.3) (layers "F.Cu" "B.Cu") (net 9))
 (via (at 68.83 54.99) (size 0.6) (drill 0.3) (layers "F.Cu" "B.Cu") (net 9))
 (segment (start 69.9008 56.0832) (end 68.83 55.0124) (width 0.25) (layer "B.Cu") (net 9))
 (segment (start 68.83 55.0124) (end 68.83 54.99) (width 0.25) (layer "B.Cu") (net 9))
 (segment (start 69.9008 63.881) (end 69.9008 56.0832) (width 0.25) (layer "B.Cu") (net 9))
 (segment (start 68.426 63.981) (end 68.4276 63.9826) (width 0.25) (layer "F.Cu") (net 1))
 (segment (start 62.7 59.0625) (end 64.0917 59.0625) (width 0.25) (layer "F.Cu") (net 1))
 (segment (start 66.7952 61.766) (end 66.7952 63.981) (width 0.25) (layer "F.Cu") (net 1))
 (segment (start 66.7952 63.981) (end 68.426 63.981) (width 0.25) (layer "F.Cu") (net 1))
 (segment (start 64.0917 59.0625) (end 66.7952 61.766) (width 0.25) (layer "F.Cu") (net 1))
 (segment (start 58.7981 60.9375) (end 62.7 60.9375) (width 0.25) (layer "F.Cu") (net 2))
 (segment (start 57.6 63.225) (end 57.6 62.1356) (width 0.25) (layer "F.Cu") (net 2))
 (segment (start 57.6 62.1356) (end 58.7981 60.9375) (width 0.25) (layer "F.Cu") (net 2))
 (segment (start 62.0058 63.225) (end 59.5 63.225) (width 0.25) (layer "F.Cu") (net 8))
 (segment (start 59.545 63.18) (end 59.5 63.225) (width 0.25) (layer "F.Cu") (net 8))
 (segment (start 64.5202 63.981) (end 62.7618 63.981) (width 0.25) (layer "F.Cu") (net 8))
 (segment (start 62.7618 63.981) (end 62.0058 63.225) (width 0.25) (layer "F.Cu") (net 8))
 (segment (start 66.7952 67.346) (end 66.6602 67.481) (width 0.25) (layer "F.Cu") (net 7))
 (segment (start 67.7164 67.3608) (end 68.4276 67.3608) (width 0.25) (layer "F.Cu") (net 7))
 (segment (start 66.7952 65.881) (end 66.7952 67.196) (width 0.25) (layer "F.Cu") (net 7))
 (segment (start 66.5226 67.481) (end 67.5962 67.481) (width 0.25) (layer "F.Cu") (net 7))
 (segment (start 66.5226 67.481) (end 66.1702 67.481) (width 0.25) (layer "F.Cu") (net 7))
 (segment (start 66.7952 67.196) (end 66.7952 67.346) (width 0.25) (layer "F.Cu") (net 7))
 (segment (start 66.6602 67.481) (end 66.5226 67.481) (width 0.25) (layer "F.Cu") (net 7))
 (segment (start 67.5962 67.481) (end 67.7164 67.3608) (width 0.25) (layer "F.Cu") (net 7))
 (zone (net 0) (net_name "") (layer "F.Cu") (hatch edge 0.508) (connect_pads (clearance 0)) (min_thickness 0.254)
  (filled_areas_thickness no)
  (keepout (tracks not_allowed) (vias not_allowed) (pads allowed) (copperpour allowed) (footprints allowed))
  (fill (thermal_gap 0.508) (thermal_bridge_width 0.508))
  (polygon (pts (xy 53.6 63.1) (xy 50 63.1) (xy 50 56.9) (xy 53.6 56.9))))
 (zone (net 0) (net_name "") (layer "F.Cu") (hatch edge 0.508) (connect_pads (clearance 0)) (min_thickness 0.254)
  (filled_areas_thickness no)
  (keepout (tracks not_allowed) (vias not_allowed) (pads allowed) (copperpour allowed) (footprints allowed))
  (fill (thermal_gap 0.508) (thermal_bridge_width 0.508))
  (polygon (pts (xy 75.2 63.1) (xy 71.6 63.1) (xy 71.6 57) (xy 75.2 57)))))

